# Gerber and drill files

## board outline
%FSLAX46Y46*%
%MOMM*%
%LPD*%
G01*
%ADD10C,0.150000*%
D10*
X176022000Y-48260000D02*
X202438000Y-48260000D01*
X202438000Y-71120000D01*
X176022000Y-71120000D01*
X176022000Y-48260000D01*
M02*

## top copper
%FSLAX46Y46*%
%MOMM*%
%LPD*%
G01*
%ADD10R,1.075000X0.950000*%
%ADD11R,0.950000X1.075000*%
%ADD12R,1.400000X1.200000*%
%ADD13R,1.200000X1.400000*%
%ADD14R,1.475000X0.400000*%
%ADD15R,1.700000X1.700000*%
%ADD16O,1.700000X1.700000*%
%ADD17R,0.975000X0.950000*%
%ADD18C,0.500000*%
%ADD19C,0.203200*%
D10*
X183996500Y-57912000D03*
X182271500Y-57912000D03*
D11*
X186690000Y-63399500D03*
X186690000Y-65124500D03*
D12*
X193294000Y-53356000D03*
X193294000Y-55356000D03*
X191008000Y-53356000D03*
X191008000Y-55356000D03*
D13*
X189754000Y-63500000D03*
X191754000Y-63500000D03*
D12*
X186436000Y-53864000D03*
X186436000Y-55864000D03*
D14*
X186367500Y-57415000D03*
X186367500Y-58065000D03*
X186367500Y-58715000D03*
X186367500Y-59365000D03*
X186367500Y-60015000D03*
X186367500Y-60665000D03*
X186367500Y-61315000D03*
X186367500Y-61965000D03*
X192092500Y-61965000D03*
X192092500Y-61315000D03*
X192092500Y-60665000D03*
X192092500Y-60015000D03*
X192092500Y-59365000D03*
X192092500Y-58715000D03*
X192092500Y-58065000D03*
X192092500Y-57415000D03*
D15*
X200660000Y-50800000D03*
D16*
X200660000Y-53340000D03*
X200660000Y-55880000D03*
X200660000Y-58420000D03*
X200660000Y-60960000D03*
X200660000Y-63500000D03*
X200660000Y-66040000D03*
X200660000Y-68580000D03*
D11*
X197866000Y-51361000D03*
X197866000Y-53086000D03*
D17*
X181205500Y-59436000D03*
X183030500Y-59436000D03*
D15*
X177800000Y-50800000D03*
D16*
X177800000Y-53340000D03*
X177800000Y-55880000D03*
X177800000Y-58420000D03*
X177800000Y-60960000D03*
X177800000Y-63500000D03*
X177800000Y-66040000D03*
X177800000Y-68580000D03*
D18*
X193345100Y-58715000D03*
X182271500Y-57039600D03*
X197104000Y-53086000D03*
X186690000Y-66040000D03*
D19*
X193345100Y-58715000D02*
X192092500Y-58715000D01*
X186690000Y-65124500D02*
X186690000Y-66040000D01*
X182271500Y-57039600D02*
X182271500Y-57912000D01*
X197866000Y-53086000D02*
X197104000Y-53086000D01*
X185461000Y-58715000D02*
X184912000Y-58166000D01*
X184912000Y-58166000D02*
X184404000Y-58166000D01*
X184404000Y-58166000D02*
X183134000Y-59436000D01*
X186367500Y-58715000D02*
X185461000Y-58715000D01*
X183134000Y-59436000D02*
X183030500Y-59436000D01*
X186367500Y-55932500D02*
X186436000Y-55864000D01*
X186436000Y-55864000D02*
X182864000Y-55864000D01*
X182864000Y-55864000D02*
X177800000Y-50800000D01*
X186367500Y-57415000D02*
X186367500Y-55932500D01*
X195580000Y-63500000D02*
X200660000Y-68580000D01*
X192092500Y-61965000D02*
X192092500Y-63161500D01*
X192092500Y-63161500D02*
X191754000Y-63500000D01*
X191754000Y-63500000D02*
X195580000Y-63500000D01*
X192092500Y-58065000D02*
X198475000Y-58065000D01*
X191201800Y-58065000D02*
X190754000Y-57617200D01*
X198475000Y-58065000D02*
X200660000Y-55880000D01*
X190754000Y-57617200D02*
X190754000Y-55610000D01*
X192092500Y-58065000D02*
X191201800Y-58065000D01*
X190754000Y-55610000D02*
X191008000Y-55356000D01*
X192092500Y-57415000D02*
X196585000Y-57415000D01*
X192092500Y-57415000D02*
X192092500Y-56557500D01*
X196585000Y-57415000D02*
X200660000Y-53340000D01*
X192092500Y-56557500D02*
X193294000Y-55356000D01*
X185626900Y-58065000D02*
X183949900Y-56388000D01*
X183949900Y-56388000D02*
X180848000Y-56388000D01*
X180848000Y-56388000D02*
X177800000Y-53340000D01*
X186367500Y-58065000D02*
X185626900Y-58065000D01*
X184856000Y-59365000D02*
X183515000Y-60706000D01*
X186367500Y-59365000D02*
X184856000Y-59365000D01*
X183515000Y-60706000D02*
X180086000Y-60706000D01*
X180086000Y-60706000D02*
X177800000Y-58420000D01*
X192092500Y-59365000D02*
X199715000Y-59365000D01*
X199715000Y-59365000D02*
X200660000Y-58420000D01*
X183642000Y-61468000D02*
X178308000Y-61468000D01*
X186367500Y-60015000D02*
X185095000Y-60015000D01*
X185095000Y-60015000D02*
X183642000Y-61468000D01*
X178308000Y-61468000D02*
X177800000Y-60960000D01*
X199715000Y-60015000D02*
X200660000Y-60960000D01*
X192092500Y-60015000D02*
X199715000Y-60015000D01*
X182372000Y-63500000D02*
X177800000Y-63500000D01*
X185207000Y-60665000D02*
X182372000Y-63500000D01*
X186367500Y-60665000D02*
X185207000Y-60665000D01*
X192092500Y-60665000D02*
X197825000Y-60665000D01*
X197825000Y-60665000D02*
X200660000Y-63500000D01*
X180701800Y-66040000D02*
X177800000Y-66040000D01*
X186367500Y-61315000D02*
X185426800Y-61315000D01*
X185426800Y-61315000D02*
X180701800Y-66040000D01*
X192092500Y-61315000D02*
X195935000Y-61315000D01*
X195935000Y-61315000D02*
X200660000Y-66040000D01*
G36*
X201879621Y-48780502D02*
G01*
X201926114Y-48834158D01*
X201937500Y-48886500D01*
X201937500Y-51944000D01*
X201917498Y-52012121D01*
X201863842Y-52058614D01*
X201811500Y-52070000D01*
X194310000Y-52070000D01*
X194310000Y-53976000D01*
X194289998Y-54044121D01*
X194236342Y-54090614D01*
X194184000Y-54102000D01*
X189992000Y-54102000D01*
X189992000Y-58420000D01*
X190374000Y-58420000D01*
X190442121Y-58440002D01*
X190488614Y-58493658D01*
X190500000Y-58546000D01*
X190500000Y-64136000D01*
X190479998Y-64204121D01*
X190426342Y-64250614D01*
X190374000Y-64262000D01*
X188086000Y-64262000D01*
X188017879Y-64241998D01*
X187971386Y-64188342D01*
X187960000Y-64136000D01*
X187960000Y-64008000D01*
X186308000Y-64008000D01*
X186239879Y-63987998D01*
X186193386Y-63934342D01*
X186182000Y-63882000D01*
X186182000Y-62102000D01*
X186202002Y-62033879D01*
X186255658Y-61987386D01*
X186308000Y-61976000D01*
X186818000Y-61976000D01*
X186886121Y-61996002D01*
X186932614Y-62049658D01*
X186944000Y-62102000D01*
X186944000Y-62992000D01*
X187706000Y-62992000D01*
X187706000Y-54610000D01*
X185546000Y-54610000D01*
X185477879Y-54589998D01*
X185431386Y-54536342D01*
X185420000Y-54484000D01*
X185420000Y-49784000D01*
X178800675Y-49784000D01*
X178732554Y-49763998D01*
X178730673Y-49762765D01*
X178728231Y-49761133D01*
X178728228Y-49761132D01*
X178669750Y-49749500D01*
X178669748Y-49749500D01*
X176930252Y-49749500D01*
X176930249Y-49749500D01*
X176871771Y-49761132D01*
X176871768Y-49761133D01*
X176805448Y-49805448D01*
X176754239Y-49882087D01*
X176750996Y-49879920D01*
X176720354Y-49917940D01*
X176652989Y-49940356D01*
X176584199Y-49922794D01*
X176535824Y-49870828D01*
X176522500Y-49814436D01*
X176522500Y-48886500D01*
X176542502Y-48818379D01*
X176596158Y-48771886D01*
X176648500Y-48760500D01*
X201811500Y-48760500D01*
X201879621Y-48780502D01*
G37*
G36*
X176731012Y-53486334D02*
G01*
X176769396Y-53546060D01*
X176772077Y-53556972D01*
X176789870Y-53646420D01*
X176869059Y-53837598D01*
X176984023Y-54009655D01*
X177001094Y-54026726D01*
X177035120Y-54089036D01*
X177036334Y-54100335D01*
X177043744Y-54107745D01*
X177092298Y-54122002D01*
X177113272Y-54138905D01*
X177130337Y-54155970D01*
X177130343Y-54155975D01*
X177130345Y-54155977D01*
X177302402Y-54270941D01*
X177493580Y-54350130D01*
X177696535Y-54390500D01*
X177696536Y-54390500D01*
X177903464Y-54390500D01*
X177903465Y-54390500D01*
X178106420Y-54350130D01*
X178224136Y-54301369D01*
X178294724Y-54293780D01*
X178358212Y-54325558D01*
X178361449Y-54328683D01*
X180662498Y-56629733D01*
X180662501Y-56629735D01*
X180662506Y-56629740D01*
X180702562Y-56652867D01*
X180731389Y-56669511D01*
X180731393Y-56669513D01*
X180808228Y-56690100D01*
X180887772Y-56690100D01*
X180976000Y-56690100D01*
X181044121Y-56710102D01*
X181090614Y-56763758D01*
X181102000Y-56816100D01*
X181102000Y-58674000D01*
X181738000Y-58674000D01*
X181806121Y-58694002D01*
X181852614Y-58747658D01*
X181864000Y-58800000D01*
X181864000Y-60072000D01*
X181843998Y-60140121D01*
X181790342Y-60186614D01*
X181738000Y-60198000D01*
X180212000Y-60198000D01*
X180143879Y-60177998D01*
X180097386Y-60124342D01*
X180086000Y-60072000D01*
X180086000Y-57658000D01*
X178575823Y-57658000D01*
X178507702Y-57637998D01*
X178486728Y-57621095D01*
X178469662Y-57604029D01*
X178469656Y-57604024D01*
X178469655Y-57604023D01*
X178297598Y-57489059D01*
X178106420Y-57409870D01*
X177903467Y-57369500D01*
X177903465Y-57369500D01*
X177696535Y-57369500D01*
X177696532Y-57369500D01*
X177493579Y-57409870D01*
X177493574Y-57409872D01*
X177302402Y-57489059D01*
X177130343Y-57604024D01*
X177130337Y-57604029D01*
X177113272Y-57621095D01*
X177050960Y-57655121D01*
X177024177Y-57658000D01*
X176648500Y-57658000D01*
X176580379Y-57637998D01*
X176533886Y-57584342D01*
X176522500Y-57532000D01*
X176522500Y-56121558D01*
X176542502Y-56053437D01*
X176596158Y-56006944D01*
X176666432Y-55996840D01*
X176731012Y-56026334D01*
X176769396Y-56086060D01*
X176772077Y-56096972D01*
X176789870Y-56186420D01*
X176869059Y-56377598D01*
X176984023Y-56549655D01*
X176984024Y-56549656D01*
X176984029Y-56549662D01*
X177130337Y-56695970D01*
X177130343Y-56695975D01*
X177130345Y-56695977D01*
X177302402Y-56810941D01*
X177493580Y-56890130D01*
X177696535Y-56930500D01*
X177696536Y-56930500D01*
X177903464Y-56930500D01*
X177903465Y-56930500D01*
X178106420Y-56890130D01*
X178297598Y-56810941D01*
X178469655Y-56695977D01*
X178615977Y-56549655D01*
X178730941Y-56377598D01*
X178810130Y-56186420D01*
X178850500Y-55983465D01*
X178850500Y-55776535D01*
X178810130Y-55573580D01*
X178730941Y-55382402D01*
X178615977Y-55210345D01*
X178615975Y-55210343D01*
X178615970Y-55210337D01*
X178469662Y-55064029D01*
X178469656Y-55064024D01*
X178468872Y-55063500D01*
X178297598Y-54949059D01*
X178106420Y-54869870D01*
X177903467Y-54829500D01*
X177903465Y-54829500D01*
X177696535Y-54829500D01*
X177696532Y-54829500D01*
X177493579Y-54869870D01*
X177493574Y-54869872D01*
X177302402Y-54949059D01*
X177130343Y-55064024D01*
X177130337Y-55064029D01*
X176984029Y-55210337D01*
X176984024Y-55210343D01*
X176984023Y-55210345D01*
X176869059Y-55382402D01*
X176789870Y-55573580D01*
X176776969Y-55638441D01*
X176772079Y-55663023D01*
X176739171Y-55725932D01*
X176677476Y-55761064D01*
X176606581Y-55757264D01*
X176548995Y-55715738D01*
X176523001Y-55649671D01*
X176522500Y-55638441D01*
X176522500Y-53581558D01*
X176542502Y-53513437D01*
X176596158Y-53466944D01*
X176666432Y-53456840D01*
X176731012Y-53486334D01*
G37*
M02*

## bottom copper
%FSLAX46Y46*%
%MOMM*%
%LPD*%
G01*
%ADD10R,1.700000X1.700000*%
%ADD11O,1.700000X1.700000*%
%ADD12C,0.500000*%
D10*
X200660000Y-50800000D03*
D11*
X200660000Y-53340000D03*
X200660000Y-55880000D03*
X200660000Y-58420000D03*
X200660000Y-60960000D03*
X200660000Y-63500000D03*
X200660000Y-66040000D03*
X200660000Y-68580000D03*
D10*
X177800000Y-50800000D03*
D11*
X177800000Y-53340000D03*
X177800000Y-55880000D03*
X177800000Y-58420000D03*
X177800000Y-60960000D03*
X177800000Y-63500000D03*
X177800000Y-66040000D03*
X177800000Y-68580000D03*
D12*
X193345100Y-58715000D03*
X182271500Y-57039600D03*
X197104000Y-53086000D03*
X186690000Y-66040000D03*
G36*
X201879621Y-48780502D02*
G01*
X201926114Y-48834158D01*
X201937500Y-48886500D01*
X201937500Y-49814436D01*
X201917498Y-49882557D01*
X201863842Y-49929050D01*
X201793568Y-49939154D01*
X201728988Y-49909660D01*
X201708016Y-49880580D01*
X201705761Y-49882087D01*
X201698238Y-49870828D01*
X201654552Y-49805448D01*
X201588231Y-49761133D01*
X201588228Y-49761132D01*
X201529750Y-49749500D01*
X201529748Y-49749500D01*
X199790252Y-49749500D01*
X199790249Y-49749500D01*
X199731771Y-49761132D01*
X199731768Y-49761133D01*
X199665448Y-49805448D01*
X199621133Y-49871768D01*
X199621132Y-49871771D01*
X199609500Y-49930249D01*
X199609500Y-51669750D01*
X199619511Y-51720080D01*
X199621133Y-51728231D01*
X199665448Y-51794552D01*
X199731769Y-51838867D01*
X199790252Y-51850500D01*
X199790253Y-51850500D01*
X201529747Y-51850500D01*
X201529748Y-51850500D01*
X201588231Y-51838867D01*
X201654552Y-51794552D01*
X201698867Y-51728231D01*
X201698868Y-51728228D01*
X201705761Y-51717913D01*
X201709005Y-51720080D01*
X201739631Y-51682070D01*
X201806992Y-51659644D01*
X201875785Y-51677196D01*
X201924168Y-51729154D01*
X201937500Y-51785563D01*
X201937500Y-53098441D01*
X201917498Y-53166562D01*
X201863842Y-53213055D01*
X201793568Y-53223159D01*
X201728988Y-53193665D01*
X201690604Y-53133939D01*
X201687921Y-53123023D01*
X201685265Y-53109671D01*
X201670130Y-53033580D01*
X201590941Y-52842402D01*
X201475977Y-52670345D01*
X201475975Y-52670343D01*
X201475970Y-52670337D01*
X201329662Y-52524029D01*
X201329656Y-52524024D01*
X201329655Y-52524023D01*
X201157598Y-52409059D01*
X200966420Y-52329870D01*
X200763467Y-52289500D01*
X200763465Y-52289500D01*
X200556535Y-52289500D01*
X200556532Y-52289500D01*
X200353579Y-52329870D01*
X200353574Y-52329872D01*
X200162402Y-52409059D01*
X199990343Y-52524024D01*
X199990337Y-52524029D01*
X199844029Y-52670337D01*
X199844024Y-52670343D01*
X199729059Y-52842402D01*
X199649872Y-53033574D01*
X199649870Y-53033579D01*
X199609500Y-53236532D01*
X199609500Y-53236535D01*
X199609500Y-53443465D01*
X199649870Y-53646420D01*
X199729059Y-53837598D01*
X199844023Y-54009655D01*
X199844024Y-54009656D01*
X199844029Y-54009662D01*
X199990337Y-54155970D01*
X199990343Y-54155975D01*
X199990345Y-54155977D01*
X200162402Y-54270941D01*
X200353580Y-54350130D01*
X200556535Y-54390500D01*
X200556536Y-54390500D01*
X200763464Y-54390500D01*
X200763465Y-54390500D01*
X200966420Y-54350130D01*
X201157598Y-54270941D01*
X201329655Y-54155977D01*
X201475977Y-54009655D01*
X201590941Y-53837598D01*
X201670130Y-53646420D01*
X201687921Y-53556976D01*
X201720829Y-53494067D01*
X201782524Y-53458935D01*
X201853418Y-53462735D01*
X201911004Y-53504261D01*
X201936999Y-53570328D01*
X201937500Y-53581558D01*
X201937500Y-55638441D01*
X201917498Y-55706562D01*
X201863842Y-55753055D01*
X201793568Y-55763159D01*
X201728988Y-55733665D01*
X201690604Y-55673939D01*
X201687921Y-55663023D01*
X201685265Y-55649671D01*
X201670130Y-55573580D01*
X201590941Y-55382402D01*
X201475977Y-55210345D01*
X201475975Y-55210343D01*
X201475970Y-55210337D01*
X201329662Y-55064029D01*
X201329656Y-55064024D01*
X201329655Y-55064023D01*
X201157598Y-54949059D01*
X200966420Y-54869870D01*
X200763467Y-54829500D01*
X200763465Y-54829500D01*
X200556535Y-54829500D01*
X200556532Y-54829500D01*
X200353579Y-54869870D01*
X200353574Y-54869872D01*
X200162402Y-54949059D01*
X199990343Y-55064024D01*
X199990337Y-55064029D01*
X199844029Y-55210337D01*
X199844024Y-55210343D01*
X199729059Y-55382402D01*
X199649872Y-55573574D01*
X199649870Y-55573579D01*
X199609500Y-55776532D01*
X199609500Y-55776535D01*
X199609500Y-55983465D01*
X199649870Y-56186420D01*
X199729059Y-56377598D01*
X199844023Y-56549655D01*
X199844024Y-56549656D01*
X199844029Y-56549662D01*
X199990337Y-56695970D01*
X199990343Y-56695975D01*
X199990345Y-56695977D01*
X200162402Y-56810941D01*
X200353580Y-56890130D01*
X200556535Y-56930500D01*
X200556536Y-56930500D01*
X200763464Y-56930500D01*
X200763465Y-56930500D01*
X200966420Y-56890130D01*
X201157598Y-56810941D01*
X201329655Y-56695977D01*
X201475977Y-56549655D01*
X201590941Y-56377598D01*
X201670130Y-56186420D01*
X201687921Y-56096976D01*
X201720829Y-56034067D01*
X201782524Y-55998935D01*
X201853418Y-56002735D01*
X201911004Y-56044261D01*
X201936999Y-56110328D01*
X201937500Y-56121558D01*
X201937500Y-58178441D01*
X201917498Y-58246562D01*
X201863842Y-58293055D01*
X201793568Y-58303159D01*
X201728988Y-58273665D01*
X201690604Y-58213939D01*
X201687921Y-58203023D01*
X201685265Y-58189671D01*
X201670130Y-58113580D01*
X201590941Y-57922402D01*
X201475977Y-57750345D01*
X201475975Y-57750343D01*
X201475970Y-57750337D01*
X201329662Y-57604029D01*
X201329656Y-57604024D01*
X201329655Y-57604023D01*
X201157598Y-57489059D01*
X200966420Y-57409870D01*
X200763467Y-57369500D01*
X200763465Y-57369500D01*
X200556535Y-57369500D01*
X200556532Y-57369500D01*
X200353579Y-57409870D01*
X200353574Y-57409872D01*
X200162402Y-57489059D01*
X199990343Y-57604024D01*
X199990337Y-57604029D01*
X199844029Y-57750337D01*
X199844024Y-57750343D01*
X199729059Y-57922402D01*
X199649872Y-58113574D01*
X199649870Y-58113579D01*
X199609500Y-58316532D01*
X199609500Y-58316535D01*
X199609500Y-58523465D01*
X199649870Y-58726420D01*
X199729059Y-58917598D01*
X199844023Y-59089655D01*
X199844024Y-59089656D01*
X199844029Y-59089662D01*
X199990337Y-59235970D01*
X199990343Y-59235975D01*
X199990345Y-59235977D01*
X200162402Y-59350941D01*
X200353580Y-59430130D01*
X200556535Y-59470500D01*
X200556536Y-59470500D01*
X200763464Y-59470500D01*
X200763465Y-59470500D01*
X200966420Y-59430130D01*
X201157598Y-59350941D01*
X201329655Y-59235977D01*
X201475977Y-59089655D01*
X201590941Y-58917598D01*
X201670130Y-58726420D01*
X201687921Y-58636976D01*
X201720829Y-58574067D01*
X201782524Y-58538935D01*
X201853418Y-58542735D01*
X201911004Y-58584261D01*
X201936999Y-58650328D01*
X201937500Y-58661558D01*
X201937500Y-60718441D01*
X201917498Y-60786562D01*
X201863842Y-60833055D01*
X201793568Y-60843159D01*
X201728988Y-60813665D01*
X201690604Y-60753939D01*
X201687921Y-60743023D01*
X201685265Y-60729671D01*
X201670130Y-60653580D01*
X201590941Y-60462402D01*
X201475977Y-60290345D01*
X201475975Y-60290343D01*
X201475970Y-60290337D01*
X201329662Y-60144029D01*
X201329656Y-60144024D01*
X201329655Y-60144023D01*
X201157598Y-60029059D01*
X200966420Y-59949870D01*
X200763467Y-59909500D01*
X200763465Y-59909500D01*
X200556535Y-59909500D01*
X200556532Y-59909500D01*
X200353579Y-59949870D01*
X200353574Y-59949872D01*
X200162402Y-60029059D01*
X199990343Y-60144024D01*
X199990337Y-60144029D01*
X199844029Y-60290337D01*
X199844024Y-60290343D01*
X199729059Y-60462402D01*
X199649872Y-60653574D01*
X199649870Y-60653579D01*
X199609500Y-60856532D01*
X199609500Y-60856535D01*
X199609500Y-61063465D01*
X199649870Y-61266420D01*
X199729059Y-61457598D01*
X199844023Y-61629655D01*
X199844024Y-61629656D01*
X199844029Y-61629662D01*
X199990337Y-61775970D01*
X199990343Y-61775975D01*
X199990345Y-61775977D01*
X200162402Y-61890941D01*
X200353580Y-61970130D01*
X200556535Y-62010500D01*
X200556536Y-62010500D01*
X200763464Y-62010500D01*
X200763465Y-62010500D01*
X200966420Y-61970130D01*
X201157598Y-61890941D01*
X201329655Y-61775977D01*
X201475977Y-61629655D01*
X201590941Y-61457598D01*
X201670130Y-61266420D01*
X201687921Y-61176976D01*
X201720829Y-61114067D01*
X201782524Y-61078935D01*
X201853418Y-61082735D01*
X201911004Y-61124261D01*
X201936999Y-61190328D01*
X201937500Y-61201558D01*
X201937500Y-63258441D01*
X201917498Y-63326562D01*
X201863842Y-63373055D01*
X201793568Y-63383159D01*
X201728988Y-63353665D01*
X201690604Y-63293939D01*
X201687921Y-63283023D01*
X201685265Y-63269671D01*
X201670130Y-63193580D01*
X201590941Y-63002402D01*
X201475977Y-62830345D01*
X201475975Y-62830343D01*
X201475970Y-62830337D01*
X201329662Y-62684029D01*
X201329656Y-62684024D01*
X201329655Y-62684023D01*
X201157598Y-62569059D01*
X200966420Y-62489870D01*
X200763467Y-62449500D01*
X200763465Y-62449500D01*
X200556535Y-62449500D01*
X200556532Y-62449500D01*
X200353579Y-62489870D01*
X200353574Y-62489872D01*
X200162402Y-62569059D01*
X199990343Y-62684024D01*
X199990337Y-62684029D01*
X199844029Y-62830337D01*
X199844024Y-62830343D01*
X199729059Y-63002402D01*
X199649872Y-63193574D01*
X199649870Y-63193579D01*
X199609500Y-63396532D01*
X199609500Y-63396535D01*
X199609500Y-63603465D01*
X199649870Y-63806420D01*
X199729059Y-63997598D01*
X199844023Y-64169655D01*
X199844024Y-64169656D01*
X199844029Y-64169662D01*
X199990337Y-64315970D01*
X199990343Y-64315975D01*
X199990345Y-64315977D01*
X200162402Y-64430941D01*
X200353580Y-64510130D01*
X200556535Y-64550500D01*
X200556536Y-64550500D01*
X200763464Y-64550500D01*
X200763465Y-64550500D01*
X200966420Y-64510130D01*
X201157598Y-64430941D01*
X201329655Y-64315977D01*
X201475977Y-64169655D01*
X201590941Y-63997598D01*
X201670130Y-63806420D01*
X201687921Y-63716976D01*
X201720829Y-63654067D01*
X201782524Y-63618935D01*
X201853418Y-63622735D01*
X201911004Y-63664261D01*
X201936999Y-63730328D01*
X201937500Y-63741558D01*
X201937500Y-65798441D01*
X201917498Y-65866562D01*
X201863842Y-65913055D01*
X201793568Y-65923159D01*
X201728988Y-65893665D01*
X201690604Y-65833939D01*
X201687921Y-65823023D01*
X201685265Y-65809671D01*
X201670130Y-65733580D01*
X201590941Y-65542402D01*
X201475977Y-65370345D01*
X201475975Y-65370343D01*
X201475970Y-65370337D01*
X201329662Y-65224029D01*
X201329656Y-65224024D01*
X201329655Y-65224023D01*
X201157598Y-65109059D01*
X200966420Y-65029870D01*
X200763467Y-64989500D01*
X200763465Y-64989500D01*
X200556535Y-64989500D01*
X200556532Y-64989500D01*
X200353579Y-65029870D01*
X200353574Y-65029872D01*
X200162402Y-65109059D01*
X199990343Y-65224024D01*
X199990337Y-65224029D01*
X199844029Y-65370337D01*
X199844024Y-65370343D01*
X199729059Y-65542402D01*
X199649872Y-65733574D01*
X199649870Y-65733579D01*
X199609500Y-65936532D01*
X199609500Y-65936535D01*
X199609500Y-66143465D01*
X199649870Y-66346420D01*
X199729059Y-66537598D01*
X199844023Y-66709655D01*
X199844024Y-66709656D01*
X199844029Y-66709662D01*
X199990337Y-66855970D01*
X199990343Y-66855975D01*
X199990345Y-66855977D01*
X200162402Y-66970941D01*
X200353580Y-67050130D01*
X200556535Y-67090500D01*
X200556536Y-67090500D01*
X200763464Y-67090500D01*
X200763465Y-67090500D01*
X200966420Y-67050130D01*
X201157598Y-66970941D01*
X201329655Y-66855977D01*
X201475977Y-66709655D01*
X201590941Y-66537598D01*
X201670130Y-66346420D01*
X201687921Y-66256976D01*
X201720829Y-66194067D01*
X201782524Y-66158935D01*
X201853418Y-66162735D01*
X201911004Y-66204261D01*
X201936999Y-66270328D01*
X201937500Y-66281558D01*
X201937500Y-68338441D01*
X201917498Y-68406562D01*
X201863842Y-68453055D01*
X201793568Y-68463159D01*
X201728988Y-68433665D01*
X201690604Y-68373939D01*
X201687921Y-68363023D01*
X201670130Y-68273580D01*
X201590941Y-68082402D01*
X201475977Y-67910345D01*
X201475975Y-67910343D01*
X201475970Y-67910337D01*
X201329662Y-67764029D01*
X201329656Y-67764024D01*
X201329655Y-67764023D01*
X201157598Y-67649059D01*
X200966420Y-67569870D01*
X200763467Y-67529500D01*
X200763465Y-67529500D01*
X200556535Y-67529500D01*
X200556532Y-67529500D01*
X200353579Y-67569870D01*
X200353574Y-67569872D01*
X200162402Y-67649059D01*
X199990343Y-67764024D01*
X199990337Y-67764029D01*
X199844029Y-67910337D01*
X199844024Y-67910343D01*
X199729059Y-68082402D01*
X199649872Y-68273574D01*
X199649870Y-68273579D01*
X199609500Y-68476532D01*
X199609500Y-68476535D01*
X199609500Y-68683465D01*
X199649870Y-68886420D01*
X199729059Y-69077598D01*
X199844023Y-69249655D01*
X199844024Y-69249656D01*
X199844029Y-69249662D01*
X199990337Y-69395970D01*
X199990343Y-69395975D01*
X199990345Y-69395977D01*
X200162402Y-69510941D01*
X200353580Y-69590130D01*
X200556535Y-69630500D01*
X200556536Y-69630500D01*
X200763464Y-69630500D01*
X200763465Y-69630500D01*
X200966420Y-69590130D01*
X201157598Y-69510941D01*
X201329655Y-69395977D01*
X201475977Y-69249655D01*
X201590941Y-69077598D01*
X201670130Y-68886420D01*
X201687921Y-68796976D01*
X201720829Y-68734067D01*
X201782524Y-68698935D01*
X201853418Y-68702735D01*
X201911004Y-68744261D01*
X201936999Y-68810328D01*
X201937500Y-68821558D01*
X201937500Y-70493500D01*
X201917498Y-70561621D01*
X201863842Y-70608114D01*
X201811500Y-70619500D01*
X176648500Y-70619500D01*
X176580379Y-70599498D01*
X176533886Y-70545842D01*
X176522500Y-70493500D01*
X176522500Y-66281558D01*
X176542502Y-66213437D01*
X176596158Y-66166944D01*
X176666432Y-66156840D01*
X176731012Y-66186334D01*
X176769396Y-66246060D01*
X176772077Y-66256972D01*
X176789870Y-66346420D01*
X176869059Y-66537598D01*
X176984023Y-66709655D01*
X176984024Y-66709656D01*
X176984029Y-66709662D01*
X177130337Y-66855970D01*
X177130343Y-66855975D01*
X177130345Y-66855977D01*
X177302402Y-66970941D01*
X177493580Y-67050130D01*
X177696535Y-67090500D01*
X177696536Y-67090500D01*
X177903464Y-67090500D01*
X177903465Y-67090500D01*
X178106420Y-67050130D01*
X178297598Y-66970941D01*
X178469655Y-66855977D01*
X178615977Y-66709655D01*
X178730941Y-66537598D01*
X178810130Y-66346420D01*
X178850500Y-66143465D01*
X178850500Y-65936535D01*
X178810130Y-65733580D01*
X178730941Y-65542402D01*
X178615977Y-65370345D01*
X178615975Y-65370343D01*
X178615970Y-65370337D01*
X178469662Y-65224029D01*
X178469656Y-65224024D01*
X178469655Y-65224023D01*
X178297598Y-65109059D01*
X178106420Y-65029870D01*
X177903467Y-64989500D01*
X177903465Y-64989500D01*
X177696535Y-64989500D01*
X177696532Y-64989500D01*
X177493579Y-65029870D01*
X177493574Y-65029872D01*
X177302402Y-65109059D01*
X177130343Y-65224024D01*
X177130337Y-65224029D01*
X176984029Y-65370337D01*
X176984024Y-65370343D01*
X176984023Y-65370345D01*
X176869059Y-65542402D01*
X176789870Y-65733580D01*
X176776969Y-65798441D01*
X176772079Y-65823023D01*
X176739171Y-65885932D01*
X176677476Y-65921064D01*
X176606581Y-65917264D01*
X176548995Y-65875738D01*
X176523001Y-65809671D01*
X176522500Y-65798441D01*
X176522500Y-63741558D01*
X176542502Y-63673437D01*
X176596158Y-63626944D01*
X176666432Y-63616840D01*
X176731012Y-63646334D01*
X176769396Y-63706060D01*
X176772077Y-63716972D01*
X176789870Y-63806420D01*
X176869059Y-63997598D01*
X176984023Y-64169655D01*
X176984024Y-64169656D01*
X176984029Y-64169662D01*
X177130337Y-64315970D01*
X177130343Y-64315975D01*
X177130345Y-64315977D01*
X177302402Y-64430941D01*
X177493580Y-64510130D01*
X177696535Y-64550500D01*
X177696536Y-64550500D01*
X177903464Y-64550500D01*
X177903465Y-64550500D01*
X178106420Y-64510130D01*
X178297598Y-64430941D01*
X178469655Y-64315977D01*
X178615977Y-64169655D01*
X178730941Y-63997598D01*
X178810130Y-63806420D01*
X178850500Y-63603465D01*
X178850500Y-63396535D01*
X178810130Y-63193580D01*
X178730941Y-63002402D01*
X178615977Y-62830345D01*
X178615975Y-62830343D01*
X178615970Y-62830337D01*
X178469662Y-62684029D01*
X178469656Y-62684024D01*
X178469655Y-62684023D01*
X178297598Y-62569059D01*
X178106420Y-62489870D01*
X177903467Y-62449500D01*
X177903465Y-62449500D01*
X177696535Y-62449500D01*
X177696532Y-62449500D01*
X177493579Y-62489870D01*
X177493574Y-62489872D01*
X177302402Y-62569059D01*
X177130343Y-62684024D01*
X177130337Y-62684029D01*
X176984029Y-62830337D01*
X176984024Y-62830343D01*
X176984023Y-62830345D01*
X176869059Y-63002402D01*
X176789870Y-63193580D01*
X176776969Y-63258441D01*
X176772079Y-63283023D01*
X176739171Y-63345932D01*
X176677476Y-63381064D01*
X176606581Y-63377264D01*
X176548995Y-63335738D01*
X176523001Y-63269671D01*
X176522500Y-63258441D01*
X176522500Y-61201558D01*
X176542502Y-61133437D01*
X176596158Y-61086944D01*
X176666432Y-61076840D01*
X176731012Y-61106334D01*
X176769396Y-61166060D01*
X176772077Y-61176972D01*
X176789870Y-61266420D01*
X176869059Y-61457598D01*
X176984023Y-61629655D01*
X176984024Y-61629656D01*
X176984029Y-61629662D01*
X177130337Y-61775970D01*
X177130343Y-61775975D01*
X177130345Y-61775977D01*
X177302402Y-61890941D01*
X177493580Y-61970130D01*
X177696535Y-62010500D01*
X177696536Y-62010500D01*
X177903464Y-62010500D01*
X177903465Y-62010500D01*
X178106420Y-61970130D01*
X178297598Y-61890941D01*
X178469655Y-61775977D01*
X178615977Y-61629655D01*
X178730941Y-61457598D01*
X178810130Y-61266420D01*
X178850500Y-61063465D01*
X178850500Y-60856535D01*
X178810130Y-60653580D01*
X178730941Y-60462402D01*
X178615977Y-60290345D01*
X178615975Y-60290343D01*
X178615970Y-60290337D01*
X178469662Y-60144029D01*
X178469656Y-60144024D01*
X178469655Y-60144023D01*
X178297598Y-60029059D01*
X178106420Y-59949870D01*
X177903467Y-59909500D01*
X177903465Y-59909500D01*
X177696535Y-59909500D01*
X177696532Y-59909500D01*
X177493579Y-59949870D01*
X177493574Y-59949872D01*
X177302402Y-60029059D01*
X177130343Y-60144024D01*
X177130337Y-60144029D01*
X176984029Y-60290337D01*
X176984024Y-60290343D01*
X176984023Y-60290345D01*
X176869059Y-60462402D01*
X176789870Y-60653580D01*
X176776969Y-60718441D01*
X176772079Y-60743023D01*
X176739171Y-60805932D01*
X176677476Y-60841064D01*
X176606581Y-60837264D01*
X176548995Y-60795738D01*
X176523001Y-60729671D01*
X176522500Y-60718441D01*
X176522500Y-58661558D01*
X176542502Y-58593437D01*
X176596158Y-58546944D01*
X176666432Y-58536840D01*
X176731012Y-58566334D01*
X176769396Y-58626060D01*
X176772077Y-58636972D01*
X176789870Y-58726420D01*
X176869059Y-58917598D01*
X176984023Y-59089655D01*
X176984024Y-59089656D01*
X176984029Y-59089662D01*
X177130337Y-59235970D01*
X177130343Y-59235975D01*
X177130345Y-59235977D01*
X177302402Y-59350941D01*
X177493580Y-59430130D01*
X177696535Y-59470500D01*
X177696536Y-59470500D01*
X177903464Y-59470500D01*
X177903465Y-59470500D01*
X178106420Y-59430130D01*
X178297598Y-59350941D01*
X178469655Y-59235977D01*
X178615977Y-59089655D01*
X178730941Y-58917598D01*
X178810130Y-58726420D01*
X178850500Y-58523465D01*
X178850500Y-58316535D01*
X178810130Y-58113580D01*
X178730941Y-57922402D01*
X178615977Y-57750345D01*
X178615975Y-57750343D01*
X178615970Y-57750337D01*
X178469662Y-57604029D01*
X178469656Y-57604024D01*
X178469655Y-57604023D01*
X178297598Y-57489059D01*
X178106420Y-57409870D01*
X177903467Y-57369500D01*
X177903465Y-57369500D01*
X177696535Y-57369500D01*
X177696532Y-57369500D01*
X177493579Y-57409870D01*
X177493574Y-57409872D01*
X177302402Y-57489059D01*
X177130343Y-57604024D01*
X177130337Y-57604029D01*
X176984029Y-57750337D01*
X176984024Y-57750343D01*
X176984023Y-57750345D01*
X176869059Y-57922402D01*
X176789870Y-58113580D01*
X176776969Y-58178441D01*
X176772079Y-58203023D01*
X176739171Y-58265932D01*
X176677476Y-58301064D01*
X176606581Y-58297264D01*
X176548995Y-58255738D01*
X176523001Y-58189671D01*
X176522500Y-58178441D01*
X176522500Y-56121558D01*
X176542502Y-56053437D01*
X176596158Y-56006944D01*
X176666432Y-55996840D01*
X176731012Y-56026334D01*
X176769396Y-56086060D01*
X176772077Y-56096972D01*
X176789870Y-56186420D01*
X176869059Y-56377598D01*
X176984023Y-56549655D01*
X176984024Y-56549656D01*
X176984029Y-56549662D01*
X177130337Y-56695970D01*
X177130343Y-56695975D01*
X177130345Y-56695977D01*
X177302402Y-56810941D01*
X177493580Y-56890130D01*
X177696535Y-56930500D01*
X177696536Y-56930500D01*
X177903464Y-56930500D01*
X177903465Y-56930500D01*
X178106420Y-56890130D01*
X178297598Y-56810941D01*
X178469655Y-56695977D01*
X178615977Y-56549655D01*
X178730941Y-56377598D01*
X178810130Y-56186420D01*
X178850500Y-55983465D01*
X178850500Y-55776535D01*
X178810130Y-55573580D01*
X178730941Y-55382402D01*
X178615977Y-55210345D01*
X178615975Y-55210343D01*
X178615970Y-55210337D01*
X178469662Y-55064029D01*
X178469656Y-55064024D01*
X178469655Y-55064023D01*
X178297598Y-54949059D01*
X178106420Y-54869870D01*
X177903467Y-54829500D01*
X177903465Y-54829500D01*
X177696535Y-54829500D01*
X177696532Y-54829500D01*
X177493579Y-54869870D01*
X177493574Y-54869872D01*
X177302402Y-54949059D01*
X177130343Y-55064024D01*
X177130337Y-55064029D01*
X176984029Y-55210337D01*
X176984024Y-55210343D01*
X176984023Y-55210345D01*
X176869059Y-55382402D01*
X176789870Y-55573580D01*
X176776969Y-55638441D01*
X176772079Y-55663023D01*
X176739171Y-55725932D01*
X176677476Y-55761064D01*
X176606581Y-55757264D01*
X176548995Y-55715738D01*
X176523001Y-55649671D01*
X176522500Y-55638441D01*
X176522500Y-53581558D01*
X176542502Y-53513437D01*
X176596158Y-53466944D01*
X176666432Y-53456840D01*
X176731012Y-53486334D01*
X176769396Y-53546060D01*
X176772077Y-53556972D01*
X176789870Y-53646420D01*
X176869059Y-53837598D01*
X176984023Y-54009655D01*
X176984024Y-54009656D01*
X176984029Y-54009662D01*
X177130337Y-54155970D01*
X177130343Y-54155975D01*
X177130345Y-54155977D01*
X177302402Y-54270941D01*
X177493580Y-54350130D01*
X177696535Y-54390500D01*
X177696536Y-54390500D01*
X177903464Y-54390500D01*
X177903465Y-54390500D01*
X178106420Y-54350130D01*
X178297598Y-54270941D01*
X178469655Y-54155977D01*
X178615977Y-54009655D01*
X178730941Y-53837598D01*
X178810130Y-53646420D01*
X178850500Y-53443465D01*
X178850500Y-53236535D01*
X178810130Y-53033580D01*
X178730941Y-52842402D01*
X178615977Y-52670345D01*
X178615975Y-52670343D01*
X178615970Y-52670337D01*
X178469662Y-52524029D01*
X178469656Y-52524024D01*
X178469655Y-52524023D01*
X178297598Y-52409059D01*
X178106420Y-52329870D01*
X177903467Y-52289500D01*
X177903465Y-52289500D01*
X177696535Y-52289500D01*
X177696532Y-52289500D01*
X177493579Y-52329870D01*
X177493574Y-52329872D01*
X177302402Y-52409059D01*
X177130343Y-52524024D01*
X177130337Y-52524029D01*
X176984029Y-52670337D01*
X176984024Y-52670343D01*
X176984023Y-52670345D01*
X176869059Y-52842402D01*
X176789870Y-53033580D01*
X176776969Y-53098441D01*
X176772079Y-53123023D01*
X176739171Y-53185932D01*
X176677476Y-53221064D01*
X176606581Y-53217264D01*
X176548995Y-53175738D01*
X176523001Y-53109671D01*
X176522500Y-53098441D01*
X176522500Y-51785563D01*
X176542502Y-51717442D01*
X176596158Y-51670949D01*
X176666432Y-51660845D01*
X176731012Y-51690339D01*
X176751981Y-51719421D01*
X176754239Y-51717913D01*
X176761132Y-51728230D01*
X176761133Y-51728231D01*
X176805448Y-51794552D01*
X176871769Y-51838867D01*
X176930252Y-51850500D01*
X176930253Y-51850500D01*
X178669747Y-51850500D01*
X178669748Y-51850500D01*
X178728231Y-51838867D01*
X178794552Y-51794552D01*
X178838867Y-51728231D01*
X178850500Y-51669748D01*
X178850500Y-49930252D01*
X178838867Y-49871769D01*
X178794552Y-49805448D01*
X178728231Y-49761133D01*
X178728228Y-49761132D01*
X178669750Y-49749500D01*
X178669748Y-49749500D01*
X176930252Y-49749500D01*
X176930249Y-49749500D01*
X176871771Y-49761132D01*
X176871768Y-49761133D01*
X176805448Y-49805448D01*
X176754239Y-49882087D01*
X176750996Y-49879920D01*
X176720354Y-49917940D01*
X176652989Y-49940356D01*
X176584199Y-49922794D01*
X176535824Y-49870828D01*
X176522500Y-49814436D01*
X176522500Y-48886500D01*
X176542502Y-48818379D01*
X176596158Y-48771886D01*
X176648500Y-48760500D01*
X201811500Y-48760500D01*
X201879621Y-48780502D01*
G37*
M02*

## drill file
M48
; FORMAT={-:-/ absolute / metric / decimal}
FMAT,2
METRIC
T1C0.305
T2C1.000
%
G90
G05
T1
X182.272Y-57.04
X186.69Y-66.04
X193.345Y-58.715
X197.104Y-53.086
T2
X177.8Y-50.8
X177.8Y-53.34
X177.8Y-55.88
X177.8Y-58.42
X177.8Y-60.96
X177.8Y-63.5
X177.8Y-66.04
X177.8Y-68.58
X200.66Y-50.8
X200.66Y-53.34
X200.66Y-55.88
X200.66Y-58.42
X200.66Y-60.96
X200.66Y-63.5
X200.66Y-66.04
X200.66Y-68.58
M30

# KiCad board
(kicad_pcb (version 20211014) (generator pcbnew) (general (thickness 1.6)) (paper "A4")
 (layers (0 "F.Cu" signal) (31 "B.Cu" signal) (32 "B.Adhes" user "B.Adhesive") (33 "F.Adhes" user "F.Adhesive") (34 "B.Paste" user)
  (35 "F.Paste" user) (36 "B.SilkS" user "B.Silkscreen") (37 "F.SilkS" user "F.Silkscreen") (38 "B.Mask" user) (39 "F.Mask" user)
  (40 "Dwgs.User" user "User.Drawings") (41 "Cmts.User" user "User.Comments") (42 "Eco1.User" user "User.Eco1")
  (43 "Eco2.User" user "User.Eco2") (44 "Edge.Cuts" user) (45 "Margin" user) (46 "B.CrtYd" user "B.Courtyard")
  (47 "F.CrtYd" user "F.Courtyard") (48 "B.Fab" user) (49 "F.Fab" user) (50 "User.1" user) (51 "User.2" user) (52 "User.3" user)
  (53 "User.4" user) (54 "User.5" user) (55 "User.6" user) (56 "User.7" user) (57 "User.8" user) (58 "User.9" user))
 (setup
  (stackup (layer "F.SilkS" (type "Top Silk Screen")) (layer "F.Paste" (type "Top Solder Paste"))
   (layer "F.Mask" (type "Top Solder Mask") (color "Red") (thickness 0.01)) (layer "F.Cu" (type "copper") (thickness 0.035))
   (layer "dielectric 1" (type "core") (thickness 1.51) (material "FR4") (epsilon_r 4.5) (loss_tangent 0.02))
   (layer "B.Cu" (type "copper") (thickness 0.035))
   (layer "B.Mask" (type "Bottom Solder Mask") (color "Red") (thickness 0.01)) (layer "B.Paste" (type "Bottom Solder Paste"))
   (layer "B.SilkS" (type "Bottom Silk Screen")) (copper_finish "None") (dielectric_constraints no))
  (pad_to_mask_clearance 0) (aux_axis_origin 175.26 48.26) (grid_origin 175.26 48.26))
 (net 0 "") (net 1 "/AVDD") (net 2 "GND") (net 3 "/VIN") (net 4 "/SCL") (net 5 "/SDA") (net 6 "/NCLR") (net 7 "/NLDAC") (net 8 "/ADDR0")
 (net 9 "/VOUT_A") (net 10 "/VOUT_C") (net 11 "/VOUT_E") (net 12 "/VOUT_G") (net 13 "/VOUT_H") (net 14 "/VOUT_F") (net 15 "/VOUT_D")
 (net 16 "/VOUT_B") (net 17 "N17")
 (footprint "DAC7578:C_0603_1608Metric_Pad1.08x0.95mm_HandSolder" (layer "F.Cu") (at 183.134 57.912 180)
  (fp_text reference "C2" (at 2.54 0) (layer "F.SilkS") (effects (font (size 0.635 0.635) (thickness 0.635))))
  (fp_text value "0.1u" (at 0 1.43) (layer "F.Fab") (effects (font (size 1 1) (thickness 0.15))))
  (pad "1" smd rect (at -0.8625 0 180) (size 1.075 0.95) (layers "F.Cu" "F.Paste" "F.Mask") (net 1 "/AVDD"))
  (pad "2" smd rect (at 0.8625 0 180) (size 1.075 0.95) (layers "F.Cu" "F.Paste" "F.Mask") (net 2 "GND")))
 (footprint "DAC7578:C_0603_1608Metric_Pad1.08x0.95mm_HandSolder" (layer "F.Cu") (at 186.69 64.262 -90)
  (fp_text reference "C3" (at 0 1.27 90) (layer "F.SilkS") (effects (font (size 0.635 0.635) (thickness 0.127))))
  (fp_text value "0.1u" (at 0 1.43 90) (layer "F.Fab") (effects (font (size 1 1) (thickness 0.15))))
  (pad "1" smd rect (at -0.8625 0 270) (size 1.075 0.95) (layers "F.Cu" "F.Paste" "F.Mask") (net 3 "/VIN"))
  (pad "2" smd rect (at 0.8625 0 270) (size 1.075 0.95) (layers "F.Cu" "F.Paste" "F.Mask") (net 2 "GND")))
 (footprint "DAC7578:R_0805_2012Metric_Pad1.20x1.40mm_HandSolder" (layer "F.Cu") (at 193.294 54.356 -90)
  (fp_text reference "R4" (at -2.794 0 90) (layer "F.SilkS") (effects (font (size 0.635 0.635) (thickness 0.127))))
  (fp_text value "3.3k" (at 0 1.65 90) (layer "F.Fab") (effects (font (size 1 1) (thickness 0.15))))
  (pad "1" smd rect (at -1 0 270) (size 1.2 1.4) (layers "F.Cu" "F.Paste" "F.Mask") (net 3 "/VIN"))
  (pad "2" smd rect (at 1 0 270) (size 1.2 1.4) (layers "F.Cu" "F.Paste" "F.Mask") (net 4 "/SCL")))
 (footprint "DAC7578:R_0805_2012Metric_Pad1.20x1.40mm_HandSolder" (layer "F.Cu") (at 191.008 54.356 -90)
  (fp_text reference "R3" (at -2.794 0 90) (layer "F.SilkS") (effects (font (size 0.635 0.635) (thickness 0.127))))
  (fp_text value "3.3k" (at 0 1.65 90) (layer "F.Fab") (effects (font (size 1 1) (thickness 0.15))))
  (pad "1" smd rect (at -1 0 270) (size 1.2 1.4) (layers "F.Cu" "F.Paste" "F.Mask") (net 3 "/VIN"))
  (pad "2" smd rect (at 1 0 270) (size 1.2 1.4) (layers "F.Cu" "F.Paste" "F.Mask") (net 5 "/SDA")))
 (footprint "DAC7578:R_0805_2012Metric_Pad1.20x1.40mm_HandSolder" (layer "F.Cu") (at 190.754 63.5)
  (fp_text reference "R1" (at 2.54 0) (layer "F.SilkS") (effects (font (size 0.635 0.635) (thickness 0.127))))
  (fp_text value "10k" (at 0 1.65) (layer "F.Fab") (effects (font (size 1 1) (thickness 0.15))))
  (pad "1" smd rect (at -1 0) (size 1.2 1.4) (layers "F.Cu" "F.Paste" "F.Mask") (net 3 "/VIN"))
  (pad "2" smd rect (at 1 0) (size 1.2 1.4) (layers "F.Cu" "F.Paste" "F.Mask") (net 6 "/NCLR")))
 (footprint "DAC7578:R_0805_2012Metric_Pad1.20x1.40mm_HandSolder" (layer "F.Cu") (at 186.436 54.864 -90)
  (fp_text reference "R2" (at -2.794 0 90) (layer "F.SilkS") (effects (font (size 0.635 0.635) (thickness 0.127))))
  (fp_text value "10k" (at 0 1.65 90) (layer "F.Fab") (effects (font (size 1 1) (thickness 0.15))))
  (pad "1" smd rect (at -1 0 270) (size 1.2 1.4) (layers "F.Cu" "F.Paste" "F.Mask") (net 3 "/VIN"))
  (pad "2" smd rect (at 1 0 270) (size 1.2 1.4) (layers "F.Cu" "F.Paste" "F.Mask") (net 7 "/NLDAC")))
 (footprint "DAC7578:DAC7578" (layer "F.Cu") (at 189.23 59.69)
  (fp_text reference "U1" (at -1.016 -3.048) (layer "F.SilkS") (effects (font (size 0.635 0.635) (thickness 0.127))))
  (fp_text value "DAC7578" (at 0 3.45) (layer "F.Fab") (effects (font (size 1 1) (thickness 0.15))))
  (pad "1" smd rect (at -2.8625 -2.275) (size 1.475 0.4) (layers "F.Cu" "F.Paste" "F.Mask") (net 7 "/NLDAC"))
  (pad "2" smd rect (at -2.8625 -1.625) (size 1.475 0.4) (layers "F.Cu" "F.Paste" "F.Mask") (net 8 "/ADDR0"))
  (pad "3" smd rect (at -2.8625 -0.975) (size 1.475 0.4) (layers "F.Cu" "F.Paste" "F.Mask") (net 1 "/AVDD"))
  (pad "4" smd rect (at -2.8625 -0.325) (size 1.475 0.4) (layers "F.Cu" "F.Paste" "F.Mask") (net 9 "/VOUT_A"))
  (pad "5" smd rect (at -2.8625 0.325) (size 1.475 0.4) (layers "F.Cu" "F.Paste" "F.Mask") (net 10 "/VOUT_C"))
  (pad "6" smd rect (at -2.8625 0.975) (size 1.475 0.4) (layers "F.Cu" "F.Paste" "F.Mask") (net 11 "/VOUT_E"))
  (pad "7" smd rect (at -2.8625 1.625) (size 1.475 0.4) (layers "F.Cu" "F.Paste" "F.Mask") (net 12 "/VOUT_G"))
  (pad "8" smd rect (at -2.8625 2.275) (size 1.475 0.4) (layers "F.Cu" "F.Paste" "F.Mask") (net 3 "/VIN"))
  (pad "9" smd rect (at 2.8625 2.275) (size 1.475 0.4) (layers "F.Cu" "F.Paste" "F.Mask") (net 6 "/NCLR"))
  (pad "10" smd rect (at 2.8625 1.625) (size 1.475 0.4) (layers "F.Cu" "F.Paste" "F.Mask") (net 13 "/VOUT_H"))
  (pad "11" smd rect (at 2.8625 0.975) (size 1.475 0.4) (layers "F.Cu" "F.Paste" "F.Mask") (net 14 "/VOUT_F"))
  (pad "12" smd rect (at 2.8625 0.325) (size 1.475 0.4) (layers "F.Cu" "F.Paste" "F.Mask") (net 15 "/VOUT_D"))
  (pad "13" smd rect (at 2.8625 -0.325) (size 1.475 0.4) (layers "F.Cu" "F.Paste" "F.Mask") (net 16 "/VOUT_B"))
  (pad "14" smd rect (at 2.8625 -0.975) (size 1.475 0.4) (layers "F.Cu" "F.Paste" "F.Mask") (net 2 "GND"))
  (pad "15" smd rect (at 2.8625 -1.625) (size 1.475 0.4) (layers "F.Cu" "F.Paste" "F.Mask") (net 5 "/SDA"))
  (pad "16" smd rect (at 2.8625 -2.275) (size 1.475 0.4) (layers "F.Cu" "F.Paste" "F.Mask") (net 4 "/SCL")))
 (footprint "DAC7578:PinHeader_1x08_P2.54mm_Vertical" (layer "F.Cu") (at 200.66 50.8)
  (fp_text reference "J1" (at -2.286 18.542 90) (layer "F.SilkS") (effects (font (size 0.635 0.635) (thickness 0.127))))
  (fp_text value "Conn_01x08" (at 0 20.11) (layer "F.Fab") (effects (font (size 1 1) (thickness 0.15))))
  (pad "1" thru_hole rect (at 0 0) (size 1.7 1.7) (drill 1) (layers *.Cu *.Mask) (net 3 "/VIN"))
  (pad "2" thru_hole oval (at 0 2.54) (size 1.7 1.7) (drill 1) (layers *.Cu *.Mask) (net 4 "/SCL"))
  (pad "3" thru_hole oval (at 0 5.08) (size 1.7 1.7) (drill 1) (layers *.Cu *.Mask) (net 5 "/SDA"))
  (pad "4" thru_hole oval (at 0 7.62) (size 1.7 1.7) (drill 1) (layers *.Cu *.Mask) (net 16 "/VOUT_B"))
  (pad "5" thru_hole oval (at 0 10.16) (size 1.7 1.7) (drill 1) (layers *.Cu *.Mask) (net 15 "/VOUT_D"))
  (pad "6" thru_hole oval (at 0 12.7) (size 1.7 1.7) (drill 1) (layers *.Cu *.Mask) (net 14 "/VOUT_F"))
  (pad "7" thru_hole oval (at 0 15.24) (size 1.7 1.7) (drill 1) (layers *.Cu *.Mask) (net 13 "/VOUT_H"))
  (pad "8" thru_hole oval (at 0 17.78) (size 1.7 1.7) (drill 1) (layers *.Cu *.Mask) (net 6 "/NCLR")))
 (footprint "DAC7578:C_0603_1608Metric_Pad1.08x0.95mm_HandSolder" (layer "F.Cu") (at 197.866 52.2235 -90)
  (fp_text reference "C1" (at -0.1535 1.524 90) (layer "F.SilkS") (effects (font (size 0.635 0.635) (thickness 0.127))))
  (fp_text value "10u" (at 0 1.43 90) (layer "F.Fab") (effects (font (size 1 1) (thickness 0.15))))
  (pad "1" smd rect (at -0.8625 0 270) (size 1.075 0.95) (layers "F.Cu" "F.Paste" "F.Mask") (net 3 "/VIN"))
  (pad "2" smd rect (at 0.8625 0 270) (size 1.075 0.95) (layers "F.Cu" "F.Paste" "F.Mask") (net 2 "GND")))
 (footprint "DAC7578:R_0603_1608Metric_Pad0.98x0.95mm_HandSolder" (layer "F.Cu") (at 182.118 59.436)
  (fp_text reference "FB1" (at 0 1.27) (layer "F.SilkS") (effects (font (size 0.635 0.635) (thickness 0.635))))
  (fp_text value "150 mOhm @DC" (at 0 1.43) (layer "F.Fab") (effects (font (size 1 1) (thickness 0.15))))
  (pad "1" smd rect (at -0.9125 0) (size 0.975 0.95) (layers "F.Cu" "F.Paste" "F.Mask") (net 3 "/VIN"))
  (pad "2" smd rect (at 0.9125 0) (size 0.975 0.95) (layers "F.Cu" "F.Paste" "F.Mask") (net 1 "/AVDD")))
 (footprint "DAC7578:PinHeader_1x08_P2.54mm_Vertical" (layer "F.Cu") (at 177.8 50.8)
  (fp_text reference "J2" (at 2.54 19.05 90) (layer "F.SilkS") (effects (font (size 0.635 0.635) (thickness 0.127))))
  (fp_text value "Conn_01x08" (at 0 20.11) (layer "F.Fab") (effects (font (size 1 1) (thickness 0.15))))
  (pad "1" thru_hole rect (at 0 0) (size 1.7 1.7) (drill 1) (layers *.Cu *.Mask) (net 7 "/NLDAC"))
  (pad "2" thru_hole oval (at 0 2.54) (size 1.7 1.7) (drill 1) (layers *.Cu *.Mask) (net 8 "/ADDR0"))
  (pad "3" thru_hole oval (at 0 5.08) (size 1.7 1.7) (drill 1) (layers *.Cu *.Mask) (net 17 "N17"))
  (pad "4" thru_hole oval (at 0 7.62) (size 1.7 1.7) (drill 1) (layers *.Cu *.Mask) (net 9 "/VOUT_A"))
  (pad "5" thru_hole oval (at 0 10.16) (size 1.7 1.7) (drill 1) (layers *.Cu *.Mask) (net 10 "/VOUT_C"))
  (pad "6" thru_hole oval (at 0 12.7) (size 1.7 1.7) (drill 1) (layers *.Cu *.Mask) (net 11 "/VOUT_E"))
  (pad "7" thru_hole oval (at 0 15.24) (size 1.7 1.7) (drill 1) (layers *.Cu *.Mask) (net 12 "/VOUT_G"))
  (pad "8" thru_hole oval (at 0 17.78) (size 1.7 1.7) (drill 1) (layers *.Cu *.Mask) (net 2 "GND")))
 (gr_rect (start 176.022 48.26) (end 202.438 71.12) (layer "Edge.Cuts") (width 0.15) (fill none))
 (segment (start 193.3451 58.715) (end 192.0925 58.715) (width 0.2032) (layer "F.Cu") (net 2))
 (segment (start 186.69 65.1245) (end 186.69 66.04) (width 0.2032) (layer "F.Cu") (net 2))
 (segment (start 182.2715 57.0396) (end 182.2715 57.912) (width 0.2032) (layer "F.Cu") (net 2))
 (segment (start 197.866 53.086) (end 197.104 53.086) (width 0.2032) (layer "F.Cu") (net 2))
 (via (at 193.3451 58.715) (size 0.5) (drill 0.305) (layers "F.Cu" "B.Cu") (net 2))
 (via (at 182.2715 57.0396) (size 0.5) (drill 0.305) (layers "F.Cu" "B.Cu") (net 2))
 (via (at 197.104 53.086) (size 0.5) (drill 0.305) (layers "F.Cu" "B.Cu") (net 2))
 (via (at 186.69 66.04) (size 0.5) (drill 0.305) (layers "F.Cu" "B.Cu") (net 2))
 (segment (start 185.461 58.715) (end 184.912 58.166) (width 0.2032) (layer "F.Cu") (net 1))
 (segment (start 184.912 58.166) (end 184.404 58.166) (width 0.2032) (layer "F.Cu") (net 1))
 (segment (start 184.404 58.166) (end 183.134 59.436) (width 0.2032) (layer "F.Cu") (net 1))
 (segment (start 186.3675 58.715) (end 185.461 58.715) (width 0.2032) (layer "F.Cu") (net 1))
 (segment (start 183.134 59.436) (end 183.0305 59.436) (width 0.2032) (layer "F.Cu") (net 1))
 (segment (start 186.3675 55.9325) (end 186.436 55.864) (width 0.2032) (layer "F.Cu") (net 7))
 (segment (start 186.436 55.864) (end 182.864 55.864) (width 0.2032) (layer "F.Cu") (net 7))
 (segment (start 182.864 55.864) (end 177.8 50.8) (width 0.2032) (layer "F.Cu") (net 7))
 (segment (start 186.3675 57.415) (end 186.3675 55.9325) (width 0.2032) (layer "F.Cu") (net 7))
 (segment (start 195.58 63.5) (end 200.66 68.58) (width 0.2032) (layer "F.Cu") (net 6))
 (segment (start 192.0925 61.965) (end 192.0925 63.1615) (width 0.2032) (layer "F.Cu") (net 6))
 (segment (start 192.0925 63.1615) (end 191.754 63.5) (width 0.2032) (layer "F.Cu") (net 6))
 (segment (start 191.754 63.5) (end 195.58 63.5) (width 0.2032) (layer "F.Cu") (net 6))
 (segment (start 192.0925 58.065) (end 198.475 58.065) (width 0.2032) (layer "F.Cu") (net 5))
 (segment (start 191.2018 58.065) (end 190.754 57.6172) (width 0.2032) (layer "F.Cu") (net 5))
 (segment (start 198.475 58.065) (end 200.66 55.88) (width 0.2032) (layer "F.Cu") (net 5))
 (segment (start 190.754 57.6172) (end 190.754 55.61) (width 0.2032) (layer "F.Cu") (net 5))
 (segment (start 192.0925 58.065) (end 191.2018 58.065) (width 0.2032) (layer "F.Cu") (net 5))
 (segment (start 190.754 55.61) (end 191.008 55.356) (width 0.2032) (layer "F.Cu") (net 5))
 (segment (start 192.0925 57.415) (end 196.585 57.415) (width 0.2032) (layer "F.Cu") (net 4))
 (segment (start 192.0925 57.415) (end 192.0925 56.5575) (width 0.2032) (layer "F.Cu") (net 4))
 (segment (start 196.585 57.415) (end 200.66 53.34) (width 0.2032) (layer "F.Cu") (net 4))
 (segment (start 192.0925 56.5575) (end 193.294 55.356) (width 0.2032) (layer "F.Cu") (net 4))
 (segment (start 185.6269 58.065) (end 183.9499 56.388) (width 0.2032) (layer "F.Cu") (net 8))
 (segment (start 183.9499 56.388) (end 180.848 56.388) (width 0.2032) (layer "F.Cu") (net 8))
 (segment (start 180.848 56.388) (end 177.8 53.34) (width 0.2032) (layer "F.Cu") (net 8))
 (segment (start 186.3675 58.065) (end 185.6269 58.065) (width 0.2032) (layer "F.Cu") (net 8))
 (segment (start 184.856 59.365) (end 183.515 60.706) (width 0.2032) (layer "F.Cu") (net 9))
 (segment (start 186.3675 59.365) (end 184.856 59.365) (width 0.2032) (layer "F.Cu") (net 9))
 (segment (start 183.515 60.706) (end 180.086 60.706) (width 0.2032) (layer "F.Cu") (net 9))
 (segment (start 180.086 60.706) (end 177.8 58.42) (width 0.2032) (layer "F.Cu") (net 9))
 (segment (start 192.0925 59.365) (end 199.715 59.365) (width 0.2032) (layer "F.Cu") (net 16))
 (segment (start 199.715 59.365) (end 200.66 58.42) (width 0.2032) (layer "F.Cu") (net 16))
 (segment (start 183.642 61.468) (end 178.308 61.468) (width 0.2032) (layer "F.Cu") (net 10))
 (segment (start 186.3675 60.015) (end 185.095 60.015) (width 0.2032) (layer "F.Cu") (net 10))
 (segment (start 185.095 60.015) (end 183.642 61.468) (width 0.2032) (layer "F.Cu") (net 10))
 (segment (start 178.308 61.468) (end 177.8 60.96) (width 0.2032) (layer "F.Cu") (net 10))
 (segment (start 199.715 60.015) (end 200.66 60.96) (width 0.2032) (layer "F.Cu") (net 15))
 (segment (start 192.0925 60.015) (end 199.715 60.015) (width 0.2032) (layer "F.Cu") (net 15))
 (segment (start 182.372 63.5) (end 177.8 63.5) (width 0.2032) (layer "F.Cu") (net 11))
 (segment (start 185.207 60.665) (end 182.372 63.5) (width 0.2032) (layer "F.Cu") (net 11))
 (segment (start 186.3675 60.665) (end 185.207 60.665) (width 0.2032) (layer "F.Cu") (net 11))
 (segment (start 192.0925 60.665) (end 197.825 60.665) (width 0.2032) (layer "F.Cu") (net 14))
 (segment (start 197.825 60.665) (end 200.66 63.5) (width 0.2032) (layer "F.Cu") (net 14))
 (segment (start 180.7018 66.04) (end 177.8 66.04) (width 0.2032) (layer "F.Cu") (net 12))
 (segment (start 186.3675 61.315) (end 185.4268 61.315) (width 0.2032) (layer "F.Cu") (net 12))
 (segment (start 185.4268 61.315) (end 180.7018 66.04) (width 0.2032) (layer "F.Cu") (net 12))
 (segment (start 192.0925 61.315) (end 195.935 61.315) (width 0.2032) (layer "F.Cu") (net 13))
 (segment (start 195.935 61.315) (end 200.66 66.04) (width 0.2032) (layer "F.Cu") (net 13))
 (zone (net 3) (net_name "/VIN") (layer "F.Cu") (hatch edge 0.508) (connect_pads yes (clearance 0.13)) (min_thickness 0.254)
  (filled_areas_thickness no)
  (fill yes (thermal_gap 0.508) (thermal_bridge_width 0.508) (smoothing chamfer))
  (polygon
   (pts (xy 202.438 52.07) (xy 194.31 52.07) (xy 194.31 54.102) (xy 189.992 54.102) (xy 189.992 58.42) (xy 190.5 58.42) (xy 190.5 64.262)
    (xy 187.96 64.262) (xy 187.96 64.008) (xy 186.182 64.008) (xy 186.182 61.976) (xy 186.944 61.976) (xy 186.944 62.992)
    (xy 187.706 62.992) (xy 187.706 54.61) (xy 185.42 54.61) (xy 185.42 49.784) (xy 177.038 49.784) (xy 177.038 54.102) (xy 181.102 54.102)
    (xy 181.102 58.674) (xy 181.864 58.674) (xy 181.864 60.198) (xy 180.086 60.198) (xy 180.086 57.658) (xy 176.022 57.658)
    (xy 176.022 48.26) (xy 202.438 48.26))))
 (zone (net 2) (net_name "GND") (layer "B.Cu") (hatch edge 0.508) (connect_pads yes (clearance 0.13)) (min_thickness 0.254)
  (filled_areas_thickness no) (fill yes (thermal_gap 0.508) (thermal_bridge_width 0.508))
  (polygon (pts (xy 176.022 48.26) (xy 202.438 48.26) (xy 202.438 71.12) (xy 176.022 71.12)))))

